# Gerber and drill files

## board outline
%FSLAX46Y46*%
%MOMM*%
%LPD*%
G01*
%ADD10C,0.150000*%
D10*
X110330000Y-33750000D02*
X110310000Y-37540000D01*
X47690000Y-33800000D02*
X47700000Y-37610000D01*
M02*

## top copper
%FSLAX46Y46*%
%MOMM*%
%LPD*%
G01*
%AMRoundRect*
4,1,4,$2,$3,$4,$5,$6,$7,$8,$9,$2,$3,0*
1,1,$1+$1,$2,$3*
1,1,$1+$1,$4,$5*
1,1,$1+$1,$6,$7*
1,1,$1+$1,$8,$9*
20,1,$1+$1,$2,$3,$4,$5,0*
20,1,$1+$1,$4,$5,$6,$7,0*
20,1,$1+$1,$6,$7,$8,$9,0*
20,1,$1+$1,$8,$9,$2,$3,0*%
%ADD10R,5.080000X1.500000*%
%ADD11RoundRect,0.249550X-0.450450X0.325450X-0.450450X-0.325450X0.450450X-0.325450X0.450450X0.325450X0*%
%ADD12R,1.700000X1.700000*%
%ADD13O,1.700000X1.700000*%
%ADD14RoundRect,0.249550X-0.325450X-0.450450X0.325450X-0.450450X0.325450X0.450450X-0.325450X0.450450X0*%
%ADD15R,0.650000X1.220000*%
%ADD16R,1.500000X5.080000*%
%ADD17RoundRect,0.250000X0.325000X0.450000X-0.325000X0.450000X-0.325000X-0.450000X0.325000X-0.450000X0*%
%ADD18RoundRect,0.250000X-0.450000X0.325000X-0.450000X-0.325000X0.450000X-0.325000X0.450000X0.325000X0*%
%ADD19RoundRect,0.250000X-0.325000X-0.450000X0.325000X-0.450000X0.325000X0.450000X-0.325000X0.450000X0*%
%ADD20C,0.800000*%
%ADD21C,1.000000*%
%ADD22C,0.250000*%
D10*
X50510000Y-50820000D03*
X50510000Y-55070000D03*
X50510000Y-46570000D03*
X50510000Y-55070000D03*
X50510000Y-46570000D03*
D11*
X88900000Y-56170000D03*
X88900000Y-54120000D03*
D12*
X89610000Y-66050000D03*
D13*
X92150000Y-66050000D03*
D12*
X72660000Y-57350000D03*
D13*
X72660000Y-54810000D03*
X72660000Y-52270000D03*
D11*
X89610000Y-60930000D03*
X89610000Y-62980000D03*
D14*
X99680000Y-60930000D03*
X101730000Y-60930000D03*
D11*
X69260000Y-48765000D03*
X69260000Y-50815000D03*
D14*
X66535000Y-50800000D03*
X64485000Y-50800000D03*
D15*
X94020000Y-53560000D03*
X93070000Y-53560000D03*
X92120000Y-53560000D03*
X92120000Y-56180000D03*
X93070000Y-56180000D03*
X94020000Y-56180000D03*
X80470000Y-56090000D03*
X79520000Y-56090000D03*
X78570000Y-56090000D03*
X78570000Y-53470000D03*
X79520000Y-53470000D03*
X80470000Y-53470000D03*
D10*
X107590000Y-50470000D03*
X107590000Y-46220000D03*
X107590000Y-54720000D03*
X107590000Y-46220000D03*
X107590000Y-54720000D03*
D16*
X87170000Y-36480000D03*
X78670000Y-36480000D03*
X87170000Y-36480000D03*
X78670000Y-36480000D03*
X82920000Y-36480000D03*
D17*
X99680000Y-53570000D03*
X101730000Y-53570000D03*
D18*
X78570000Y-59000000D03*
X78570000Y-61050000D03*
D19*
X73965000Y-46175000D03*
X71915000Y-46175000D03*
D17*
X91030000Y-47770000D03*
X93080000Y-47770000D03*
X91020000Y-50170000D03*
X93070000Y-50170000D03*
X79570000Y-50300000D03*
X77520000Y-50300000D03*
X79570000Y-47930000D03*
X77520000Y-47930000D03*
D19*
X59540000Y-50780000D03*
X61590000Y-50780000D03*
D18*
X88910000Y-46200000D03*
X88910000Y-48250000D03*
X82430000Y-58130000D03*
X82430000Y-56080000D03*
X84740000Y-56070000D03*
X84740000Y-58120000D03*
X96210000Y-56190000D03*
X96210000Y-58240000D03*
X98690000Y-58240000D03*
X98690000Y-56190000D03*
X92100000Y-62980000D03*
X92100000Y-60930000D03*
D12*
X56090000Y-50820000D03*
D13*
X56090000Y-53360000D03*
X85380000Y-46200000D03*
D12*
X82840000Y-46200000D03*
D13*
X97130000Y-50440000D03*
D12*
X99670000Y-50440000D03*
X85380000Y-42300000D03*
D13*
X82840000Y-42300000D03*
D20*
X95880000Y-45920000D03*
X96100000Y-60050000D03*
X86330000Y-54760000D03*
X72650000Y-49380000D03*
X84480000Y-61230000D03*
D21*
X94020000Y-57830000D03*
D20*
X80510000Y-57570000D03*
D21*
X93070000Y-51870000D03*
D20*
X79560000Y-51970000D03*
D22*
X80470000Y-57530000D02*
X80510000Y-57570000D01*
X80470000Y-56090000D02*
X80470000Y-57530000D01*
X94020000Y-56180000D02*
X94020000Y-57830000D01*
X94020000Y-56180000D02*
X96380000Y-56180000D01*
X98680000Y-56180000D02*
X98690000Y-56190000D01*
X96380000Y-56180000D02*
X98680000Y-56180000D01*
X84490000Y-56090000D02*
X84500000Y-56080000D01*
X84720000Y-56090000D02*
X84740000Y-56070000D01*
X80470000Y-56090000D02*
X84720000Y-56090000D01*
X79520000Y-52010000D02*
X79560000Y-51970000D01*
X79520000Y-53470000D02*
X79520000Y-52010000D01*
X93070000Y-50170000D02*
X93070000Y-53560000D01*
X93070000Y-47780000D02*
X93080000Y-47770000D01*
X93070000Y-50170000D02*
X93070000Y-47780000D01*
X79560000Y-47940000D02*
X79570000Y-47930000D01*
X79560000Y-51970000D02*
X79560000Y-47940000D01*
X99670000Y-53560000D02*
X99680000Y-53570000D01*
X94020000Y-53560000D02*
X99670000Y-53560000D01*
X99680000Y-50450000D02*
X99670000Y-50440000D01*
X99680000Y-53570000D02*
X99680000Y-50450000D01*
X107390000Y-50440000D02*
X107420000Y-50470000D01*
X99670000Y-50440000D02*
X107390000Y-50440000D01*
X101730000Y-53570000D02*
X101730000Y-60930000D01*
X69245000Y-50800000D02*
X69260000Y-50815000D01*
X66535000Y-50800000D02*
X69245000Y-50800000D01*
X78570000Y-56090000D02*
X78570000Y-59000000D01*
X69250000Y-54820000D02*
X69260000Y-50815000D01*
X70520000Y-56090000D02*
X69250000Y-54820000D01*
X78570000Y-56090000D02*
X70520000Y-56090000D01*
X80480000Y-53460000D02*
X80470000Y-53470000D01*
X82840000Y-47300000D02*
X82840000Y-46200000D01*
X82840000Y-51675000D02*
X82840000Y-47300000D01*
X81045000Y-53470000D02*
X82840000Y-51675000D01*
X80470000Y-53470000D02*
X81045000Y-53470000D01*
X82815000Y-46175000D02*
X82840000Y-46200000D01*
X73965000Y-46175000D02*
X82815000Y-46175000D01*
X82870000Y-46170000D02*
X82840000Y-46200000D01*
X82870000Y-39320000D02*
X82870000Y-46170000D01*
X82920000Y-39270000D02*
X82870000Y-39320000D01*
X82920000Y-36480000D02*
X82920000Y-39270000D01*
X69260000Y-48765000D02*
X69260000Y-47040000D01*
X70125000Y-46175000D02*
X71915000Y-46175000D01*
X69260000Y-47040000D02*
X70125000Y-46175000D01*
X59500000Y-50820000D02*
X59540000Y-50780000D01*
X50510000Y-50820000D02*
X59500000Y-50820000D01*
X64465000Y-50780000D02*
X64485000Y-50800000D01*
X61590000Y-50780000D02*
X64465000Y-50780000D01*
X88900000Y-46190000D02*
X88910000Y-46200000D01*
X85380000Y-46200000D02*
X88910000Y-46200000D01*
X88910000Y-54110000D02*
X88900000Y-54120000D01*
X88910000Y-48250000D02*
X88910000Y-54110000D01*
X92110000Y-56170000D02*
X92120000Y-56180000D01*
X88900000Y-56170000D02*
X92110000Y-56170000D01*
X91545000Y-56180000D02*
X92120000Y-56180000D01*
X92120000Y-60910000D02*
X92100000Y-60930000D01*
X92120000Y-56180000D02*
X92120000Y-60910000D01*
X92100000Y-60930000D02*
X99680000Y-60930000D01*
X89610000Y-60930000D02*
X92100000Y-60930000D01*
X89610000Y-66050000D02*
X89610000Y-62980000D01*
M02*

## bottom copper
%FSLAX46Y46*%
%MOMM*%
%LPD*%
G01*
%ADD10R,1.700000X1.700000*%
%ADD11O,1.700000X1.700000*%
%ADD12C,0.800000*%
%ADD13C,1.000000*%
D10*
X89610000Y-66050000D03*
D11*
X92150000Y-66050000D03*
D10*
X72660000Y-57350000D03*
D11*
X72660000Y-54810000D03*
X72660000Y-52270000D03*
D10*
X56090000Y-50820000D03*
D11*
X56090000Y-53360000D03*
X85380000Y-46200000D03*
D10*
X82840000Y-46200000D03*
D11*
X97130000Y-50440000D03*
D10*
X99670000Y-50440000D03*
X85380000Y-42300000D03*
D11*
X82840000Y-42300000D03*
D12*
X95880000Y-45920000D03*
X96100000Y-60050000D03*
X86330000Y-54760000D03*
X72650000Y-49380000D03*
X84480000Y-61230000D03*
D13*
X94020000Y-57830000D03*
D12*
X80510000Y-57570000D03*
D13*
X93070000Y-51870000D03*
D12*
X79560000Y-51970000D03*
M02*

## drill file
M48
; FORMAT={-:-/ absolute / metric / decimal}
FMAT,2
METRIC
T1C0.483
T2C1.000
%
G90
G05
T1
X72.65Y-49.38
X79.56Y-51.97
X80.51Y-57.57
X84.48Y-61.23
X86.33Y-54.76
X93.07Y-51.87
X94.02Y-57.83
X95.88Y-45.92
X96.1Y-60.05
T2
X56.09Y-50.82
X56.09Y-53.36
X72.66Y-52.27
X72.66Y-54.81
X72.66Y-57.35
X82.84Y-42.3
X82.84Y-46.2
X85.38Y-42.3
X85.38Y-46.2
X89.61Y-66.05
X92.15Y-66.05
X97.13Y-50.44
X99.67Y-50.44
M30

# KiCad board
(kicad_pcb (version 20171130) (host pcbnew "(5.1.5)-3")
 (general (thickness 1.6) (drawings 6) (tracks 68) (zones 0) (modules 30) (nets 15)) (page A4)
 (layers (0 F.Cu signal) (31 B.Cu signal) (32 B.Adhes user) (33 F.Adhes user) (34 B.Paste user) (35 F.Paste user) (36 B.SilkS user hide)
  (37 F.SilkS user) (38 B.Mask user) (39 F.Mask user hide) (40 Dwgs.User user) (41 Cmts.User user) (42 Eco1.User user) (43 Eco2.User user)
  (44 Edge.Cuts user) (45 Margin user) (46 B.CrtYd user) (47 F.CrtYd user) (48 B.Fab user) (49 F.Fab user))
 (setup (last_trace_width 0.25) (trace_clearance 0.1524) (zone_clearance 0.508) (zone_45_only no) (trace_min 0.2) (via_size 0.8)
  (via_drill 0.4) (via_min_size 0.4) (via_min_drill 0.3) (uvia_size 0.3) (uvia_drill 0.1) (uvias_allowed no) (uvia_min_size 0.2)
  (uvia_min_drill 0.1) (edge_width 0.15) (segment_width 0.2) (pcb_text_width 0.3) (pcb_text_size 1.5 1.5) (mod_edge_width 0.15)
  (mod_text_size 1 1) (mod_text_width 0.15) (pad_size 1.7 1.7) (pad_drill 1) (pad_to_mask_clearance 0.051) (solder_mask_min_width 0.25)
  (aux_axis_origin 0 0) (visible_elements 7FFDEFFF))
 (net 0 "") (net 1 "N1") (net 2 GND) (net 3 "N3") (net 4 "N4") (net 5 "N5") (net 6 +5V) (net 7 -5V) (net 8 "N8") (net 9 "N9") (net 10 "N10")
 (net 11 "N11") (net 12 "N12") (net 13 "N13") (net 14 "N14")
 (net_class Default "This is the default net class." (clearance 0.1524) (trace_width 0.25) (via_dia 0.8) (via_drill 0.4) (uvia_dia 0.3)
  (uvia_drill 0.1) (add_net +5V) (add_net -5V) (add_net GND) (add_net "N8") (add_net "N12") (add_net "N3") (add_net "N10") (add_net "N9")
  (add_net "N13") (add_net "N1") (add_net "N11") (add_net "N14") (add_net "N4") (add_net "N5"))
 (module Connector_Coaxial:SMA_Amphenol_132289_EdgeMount (layer F.Cu) (at 50.51 50.82 180)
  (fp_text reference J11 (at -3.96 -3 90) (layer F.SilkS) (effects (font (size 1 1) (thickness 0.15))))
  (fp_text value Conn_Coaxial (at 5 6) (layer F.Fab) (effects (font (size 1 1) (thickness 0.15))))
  (pad 1 smd rect (at 0 0 270) (size 1.5 5.08) (layers F.Cu F.Paste F.Mask) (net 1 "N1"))
  (pad 2 smd rect (at 0 -4.25 270) (size 1.5 5.08) (layers F.Cu F.Paste F.Mask) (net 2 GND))
  (pad 2 smd rect (at 0 4.25 270) (size 1.5 5.08) (layers F.Cu F.Paste F.Mask) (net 2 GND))
  (pad 2 smd rect (at 0 -4.25 270) (size 1.5 5.08) (layers F.Cu B.Paste B.Mask) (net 2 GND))
  (pad 2 smd rect (at 0 4.25 270) (size 1.5 5.08) (layers F.Cu B.Paste B.Mask) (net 2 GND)))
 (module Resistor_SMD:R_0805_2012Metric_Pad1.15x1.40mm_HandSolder (layer F.Cu) (at 88.9 55.145 270)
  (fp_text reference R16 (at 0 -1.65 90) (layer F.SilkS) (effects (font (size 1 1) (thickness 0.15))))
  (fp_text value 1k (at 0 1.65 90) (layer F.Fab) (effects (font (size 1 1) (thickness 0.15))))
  (pad 2 smd roundrect (at 1.025 0 270) (size 1.15 1.4) (layers F.Cu F.Paste F.Mask) (roundrect_rratio 0.217) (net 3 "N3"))
  (pad 1 smd roundrect (at -1.025 0 270) (size 1.15 1.4) (layers F.Cu F.Paste F.Mask) (roundrect_rratio 0.217) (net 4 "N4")))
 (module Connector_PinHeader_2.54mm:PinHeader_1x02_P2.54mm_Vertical (layer F.Cu) (at 89.61 66.05 90)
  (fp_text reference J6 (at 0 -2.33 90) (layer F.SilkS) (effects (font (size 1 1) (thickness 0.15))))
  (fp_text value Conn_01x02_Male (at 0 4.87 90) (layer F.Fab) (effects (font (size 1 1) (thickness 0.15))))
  (pad 1 thru_hole rect (at 0 0 90) (size 1.7 1.7) (drill 1) (layers *.Cu *.Mask) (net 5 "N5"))
  (pad 2 thru_hole oval (at 0 2.54 90) (size 1.7 1.7) (drill 1) (layers *.Cu *.Mask) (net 2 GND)))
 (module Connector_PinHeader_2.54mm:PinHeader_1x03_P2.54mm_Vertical (layer F.Cu) (at 72.66 57.35 180)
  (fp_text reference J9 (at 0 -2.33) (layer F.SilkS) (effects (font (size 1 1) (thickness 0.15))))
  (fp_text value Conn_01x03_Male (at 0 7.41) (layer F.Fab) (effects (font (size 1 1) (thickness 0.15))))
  (pad 1 thru_hole rect (at 0 0 180) (size 1.7 1.7) (drill 1) (layers *.Mask B.Cu) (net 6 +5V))
  (pad 2 thru_hole oval (at 0 2.54 180) (size 1.7 1.7) (drill 1) (layers *.Cu *.Mask) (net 2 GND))
  (pad 3 thru_hole oval (at 0 5.08 180) (size 1.7 1.7) (drill 1) (layers *.Mask B.Cu) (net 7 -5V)))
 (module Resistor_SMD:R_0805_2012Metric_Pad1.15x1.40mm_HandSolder (layer F.Cu) (at 89.61 61.955 270)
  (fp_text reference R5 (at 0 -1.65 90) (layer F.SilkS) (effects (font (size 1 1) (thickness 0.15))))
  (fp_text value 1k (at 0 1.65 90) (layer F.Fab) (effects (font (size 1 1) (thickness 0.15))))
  (pad 1 smd roundrect (at -1.025 0 270) (size 1.15 1.4) (layers F.Cu F.Paste F.Mask) (roundrect_rratio 0.217) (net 3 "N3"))
  (pad 2 smd roundrect (at 1.025 0 270) (size 1.15 1.4) (layers F.Cu F.Paste F.Mask) (roundrect_rratio 0.217) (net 5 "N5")))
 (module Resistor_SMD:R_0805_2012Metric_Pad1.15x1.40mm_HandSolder (layer F.Cu) (at 100.705 60.93)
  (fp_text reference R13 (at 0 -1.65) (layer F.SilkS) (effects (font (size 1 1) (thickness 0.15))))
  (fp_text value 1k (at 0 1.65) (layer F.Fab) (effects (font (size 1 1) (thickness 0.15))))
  (pad 1 smd roundrect (at -1.025 0) (size 1.15 1.4) (layers F.Cu F.Paste F.Mask) (roundrect_rratio 0.217) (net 3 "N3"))
  (pad 2 smd roundrect (at 1.025 0) (size 1.15 1.4) (layers F.Cu F.Paste F.Mask) (roundrect_rratio 0.217) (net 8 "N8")))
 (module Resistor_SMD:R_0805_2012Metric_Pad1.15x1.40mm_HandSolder (layer F.Cu) (at 69.26 49.79 270)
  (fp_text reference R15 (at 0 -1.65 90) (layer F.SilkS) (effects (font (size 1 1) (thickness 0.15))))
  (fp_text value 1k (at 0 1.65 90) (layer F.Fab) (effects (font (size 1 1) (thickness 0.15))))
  (pad 1 smd roundrect (at -1.025 0 270) (size 1.15 1.4) (layers F.Cu F.Paste F.Mask) (roundrect_rratio 0.217) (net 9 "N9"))
  (pad 2 smd roundrect (at 1.025 0 270) (size 1.15 1.4) (layers F.Cu F.Paste F.Mask) (roundrect_rratio 0.217) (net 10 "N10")))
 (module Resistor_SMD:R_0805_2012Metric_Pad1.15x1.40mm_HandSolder (layer F.Cu) (at 65.51 50.8)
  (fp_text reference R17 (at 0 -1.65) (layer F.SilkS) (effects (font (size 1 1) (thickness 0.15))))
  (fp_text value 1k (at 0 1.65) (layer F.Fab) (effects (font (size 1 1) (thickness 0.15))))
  (pad 2 smd roundrect (at 1.025 0) (size 1.15 1.4) (layers F.Cu F.Paste F.Mask) (roundrect_rratio 0.217) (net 10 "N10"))
  (pad 1 smd roundrect (at -1.025 0) (size 1.15 1.4) (layers F.Cu F.Paste F.Mask) (roundrect_rratio 0.217) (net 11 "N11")))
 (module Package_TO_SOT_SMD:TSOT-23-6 (layer F.Cu) (at 93.07 54.87 270)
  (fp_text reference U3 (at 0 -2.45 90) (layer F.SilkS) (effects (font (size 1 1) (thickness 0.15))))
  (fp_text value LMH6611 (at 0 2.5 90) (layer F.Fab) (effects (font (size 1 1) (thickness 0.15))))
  (pad 1 smd rect (at -1.31 -0.95 270) (size 1.22 0.65) (layers F.Cu F.Paste F.Mask) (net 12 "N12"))
  (pad 2 smd rect (at -1.31 0 270) (size 1.22 0.65) (layers F.Cu F.Paste F.Mask) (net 7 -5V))
  (pad 3 smd rect (at -1.31 0.95 270) (size 1.22 0.65) (layers F.Cu F.Paste F.Mask) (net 2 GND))
  (pad 4 smd rect (at 1.31 0.95 270) (size 1.22 0.65) (layers F.Cu F.Paste F.Mask) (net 3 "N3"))
  (pad 5 smd rect (at 1.31 0 270) (size 1.22 0.65) (layers F.Cu F.Paste F.Mask))
  (pad 6 smd rect (at 1.31 -0.95 270) (size 1.22 0.65) (layers F.Cu F.Paste F.Mask) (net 6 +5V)))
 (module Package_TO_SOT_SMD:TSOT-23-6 (layer F.Cu) (at 79.52 54.78 270)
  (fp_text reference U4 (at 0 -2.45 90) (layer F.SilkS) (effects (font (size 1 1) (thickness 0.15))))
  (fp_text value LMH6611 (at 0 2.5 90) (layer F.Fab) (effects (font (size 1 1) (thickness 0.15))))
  (pad 6 smd rect (at 1.31 -0.95 270) (size 1.22 0.65) (layers F.Cu F.Paste F.Mask) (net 6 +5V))
  (pad 5 smd rect (at 1.31 0 270) (size 1.22 0.65) (layers F.Cu F.Paste F.Mask))
  (pad 4 smd rect (at 1.31 0.95 270) (size 1.22 0.65) (layers F.Cu F.Paste F.Mask) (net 10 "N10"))
  (pad 3 smd rect (at -1.31 0.95 270) (size 1.22 0.65) (layers F.Cu F.Paste F.Mask) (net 2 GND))
  (pad 2 smd rect (at -1.31 0 270) (size 1.22 0.65) (layers F.Cu F.Paste F.Mask) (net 7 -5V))
  (pad 1 smd rect (at -1.31 -0.95 270) (size 1.22 0.65) (layers F.Cu F.Paste F.Mask) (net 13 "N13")))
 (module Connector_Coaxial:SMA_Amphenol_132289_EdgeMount (layer F.Cu) (at 107.59 50.47)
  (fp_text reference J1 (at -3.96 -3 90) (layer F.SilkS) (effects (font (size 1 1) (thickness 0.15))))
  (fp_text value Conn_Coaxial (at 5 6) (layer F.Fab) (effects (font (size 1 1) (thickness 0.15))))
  (pad 1 smd rect (at 0 0 90) (size 1.5 5.08) (layers F.Cu F.Paste F.Mask) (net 12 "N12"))
  (pad 2 smd rect (at 0 -4.25 90) (size 1.5 5.08) (layers F.Cu F.Paste F.Mask) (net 2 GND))
  (pad 2 smd rect (at 0 4.25 90) (size 1.5 5.08) (layers F.Cu F.Paste F.Mask) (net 2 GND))
  (pad 2 smd rect (at 0 -4.25 90) (size 1.5 5.08) (layers F.Cu B.Paste B.Mask) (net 2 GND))
  (pad 2 smd rect (at 0 4.25 90) (size 1.5 5.08) (layers F.Cu B.Paste B.Mask) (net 2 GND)))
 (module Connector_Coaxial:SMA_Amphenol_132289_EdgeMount (layer F.Cu) (at 82.92 36.48 90)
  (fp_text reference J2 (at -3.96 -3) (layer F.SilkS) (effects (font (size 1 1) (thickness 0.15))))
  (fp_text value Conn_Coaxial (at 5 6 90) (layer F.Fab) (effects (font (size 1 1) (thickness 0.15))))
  (pad 2 smd rect (at 0 4.25 180) (size 1.5 5.08) (layers F.Cu B.Paste B.Mask) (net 2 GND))
  (pad 2 smd rect (at 0 -4.25 180) (size 1.5 5.08) (layers F.Cu B.Paste B.Mask) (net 2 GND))
  (pad 2 smd rect (at 0 4.25 180) (size 1.5 5.08) (layers F.Cu F.Paste F.Mask) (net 2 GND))
  (pad 2 smd rect (at 0 -4.25 180) (size 1.5 5.08) (layers F.Cu F.Paste F.Mask) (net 2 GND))
  (pad 1 smd rect (at 0 0 180) (size 1.5 5.08) (layers F.Cu F.Paste F.Mask) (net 13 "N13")))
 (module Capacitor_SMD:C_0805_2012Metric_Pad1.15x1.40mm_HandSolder (layer F.Cu) (at 100.705 53.57 180)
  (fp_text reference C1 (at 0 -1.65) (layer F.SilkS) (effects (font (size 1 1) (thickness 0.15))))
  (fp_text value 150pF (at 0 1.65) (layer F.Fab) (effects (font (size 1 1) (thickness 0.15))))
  (pad 2 smd roundrect (at 1.025 0 180) (size 1.15 1.4) (layers F.Cu F.Paste F.Mask) (roundrect_rratio 0.217391) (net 12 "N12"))
  (pad 1 smd roundrect (at -1.025 0 180) (size 1.15 1.4) (layers F.Cu F.Paste F.Mask) (roundrect_rratio 0.217391) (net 8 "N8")))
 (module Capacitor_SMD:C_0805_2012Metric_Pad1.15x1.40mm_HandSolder (layer F.Cu) (at 78.57 60.025 270)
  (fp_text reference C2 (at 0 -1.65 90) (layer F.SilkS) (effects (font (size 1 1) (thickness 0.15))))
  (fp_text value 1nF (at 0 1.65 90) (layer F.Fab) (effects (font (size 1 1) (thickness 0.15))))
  (pad 1 smd roundrect (at -1.025 0 270) (size 1.15 1.4) (layers F.Cu F.Paste F.Mask) (roundrect_rratio 0.217391) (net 10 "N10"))
  (pad 2 smd roundrect (at 1.025 0 270) (size 1.15 1.4) (layers F.Cu F.Paste F.Mask) (roundrect_rratio 0.217391) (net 2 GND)))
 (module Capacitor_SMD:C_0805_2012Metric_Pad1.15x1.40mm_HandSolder (layer F.Cu) (at 72.94 46.175)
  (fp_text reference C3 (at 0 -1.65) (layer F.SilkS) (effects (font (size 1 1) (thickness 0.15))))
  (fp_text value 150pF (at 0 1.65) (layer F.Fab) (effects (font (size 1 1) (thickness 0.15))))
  (pad 2 smd roundrect (at 1.025 0) (size 1.15 1.4) (layers F.Cu F.Paste F.Mask) (roundrect_rratio 0.217391) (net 13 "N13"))
  (pad 1 smd roundrect (at -1.025 0) (size 1.15 1.4) (layers F.Cu F.Paste F.Mask) (roundrect_rratio 0.217391) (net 9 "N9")))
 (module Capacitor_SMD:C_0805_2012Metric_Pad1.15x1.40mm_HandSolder (layer F.Cu) (at 92.055 47.77 180)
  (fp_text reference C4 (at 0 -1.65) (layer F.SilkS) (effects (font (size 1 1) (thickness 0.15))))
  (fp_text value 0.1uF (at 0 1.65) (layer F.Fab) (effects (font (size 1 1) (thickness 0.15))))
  (pad 2 smd roundrect (at 1.025 0 180) (size 1.15 1.4) (layers F.Cu F.Paste F.Mask) (roundrect_rratio 0.217391) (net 2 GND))
  (pad 1 smd roundrect (at -1.025 0 180) (size 1.15 1.4) (layers F.Cu F.Paste F.Mask) (roundrect_rratio 0.217391) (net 7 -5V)))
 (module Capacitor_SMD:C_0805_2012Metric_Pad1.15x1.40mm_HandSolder (layer F.Cu) (at 92.045 50.17 180)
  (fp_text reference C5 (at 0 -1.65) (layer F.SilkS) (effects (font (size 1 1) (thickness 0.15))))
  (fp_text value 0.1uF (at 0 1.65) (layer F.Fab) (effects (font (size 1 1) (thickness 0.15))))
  (pad 2 smd roundrect (at 1.025 0 180) (size 1.15 1.4) (layers F.Cu F.Paste F.Mask) (roundrect_rratio 0.217391) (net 2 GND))
  (pad 1 smd roundrect (at -1.025 0 180) (size 1.15 1.4) (layers F.Cu F.Paste F.Mask) (roundrect_rratio 0.217391) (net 7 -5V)))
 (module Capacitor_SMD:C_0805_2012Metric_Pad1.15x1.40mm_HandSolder (layer F.Cu) (at 78.545 50.3 180)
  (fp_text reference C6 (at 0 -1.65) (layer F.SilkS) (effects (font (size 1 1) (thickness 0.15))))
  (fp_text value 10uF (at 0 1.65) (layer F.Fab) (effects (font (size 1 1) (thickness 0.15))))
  (pad 1 smd roundrect (at -1.025 0 180) (size 1.15 1.4) (layers F.Cu F.Paste F.Mask) (roundrect_rratio 0.217391) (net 7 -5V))
  (pad 2 smd roundrect (at 1.025 0 180) (size 1.15 1.4) (layers F.Cu F.Paste F.Mask) (roundrect_rratio 0.217391) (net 2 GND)))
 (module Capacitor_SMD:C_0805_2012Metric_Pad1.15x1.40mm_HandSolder (layer F.Cu) (at 78.545 47.93 180)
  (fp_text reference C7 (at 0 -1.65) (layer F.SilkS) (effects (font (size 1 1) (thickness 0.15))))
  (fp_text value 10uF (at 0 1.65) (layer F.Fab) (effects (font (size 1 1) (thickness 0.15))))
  (pad 1 smd roundrect (at -1.025 0 180) (size 1.15 1.4) (layers F.Cu F.Paste F.Mask) (roundrect_rratio 0.217391) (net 7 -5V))
  (pad 2 smd roundrect (at 1.025 0 180) (size 1.15 1.4) (layers F.Cu F.Paste F.Mask) (roundrect_rratio 0.217391) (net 2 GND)))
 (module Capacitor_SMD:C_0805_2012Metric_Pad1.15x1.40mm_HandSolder (layer F.Cu) (at 60.565 50.78)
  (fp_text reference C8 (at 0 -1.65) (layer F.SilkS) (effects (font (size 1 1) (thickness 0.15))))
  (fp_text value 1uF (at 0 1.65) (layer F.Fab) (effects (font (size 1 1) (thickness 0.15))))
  (pad 1 smd roundrect (at -1.025 0) (size 1.15 1.4) (layers F.Cu F.Paste F.Mask) (roundrect_rratio 0.217391) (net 1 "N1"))
  (pad 2 smd roundrect (at 1.025 0) (size 1.15 1.4) (layers F.Cu F.Paste F.Mask) (roundrect_rratio 0.217391) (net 11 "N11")))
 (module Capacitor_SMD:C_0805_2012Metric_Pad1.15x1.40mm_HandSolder (layer F.Cu) (at 88.91 47.225 270)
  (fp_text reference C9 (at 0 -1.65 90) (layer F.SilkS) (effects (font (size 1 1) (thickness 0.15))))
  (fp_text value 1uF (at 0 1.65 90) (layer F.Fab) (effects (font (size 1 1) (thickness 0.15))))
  (pad 1 smd roundrect (at -1.025 0 270) (size 1.15 1.4) (layers F.Cu F.Paste F.Mask) (roundrect_rratio 0.217391) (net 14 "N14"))
  (pad 2 smd roundrect (at 1.025 0 270) (size 1.15 1.4) (layers F.Cu F.Paste F.Mask) (roundrect_rratio 0.217391) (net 4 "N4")))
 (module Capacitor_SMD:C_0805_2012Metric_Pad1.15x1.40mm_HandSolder (layer F.Cu) (at 82.43 57.105 270)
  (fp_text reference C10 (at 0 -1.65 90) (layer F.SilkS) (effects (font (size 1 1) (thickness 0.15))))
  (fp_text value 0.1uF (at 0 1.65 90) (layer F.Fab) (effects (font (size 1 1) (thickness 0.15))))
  (pad 2 smd roundrect (at 1.025 0 270) (size 1.15 1.4) (layers F.Cu F.Paste F.Mask) (roundrect_rratio 0.217391) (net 2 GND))
  (pad 1 smd roundrect (at -1.025 0 270) (size 1.15 1.4) (layers F.Cu F.Paste F.Mask) (roundrect_rratio 0.217391) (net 6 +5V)))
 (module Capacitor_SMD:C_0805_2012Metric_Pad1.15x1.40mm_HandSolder (layer F.Cu) (at 84.74 57.095 270)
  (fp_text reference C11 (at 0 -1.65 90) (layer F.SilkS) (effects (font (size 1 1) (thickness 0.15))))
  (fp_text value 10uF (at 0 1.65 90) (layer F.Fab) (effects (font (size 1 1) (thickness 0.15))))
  (pad 1 smd roundrect (at -1.025 0 270) (size 1.15 1.4) (layers F.Cu F.Paste F.Mask) (roundrect_rratio 0.217391) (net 6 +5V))
  (pad 2 smd roundrect (at 1.025 0 270) (size 1.15 1.4) (layers F.Cu F.Paste F.Mask) (roundrect_rratio 0.217391) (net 2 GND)))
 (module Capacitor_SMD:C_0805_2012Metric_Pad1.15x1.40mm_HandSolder (layer F.Cu) (at 96.21 57.215 270)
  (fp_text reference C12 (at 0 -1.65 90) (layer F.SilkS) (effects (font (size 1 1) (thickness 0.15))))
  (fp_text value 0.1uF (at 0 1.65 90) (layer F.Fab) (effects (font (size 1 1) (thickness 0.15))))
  (pad 1 smd roundrect (at -1.025 0 270) (size 1.15 1.4) (layers F.Cu F.Paste F.Mask) (roundrect_rratio 0.217391) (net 6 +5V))
  (pad 2 smd roundrect (at 1.025 0 270) (size 1.15 1.4) (layers F.Cu F.Paste F.Mask) (roundrect_rratio 0.217391) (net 2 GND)))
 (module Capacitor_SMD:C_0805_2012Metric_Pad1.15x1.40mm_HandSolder (layer F.Cu) (at 98.69 57.215 270)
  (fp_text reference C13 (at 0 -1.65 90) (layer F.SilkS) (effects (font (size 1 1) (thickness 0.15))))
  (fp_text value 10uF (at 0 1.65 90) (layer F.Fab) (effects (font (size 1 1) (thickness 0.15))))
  (pad 2 smd roundrect (at 1.025 0 270) (size 1.15 1.4) (layers F.Cu F.Paste F.Mask) (roundrect_rratio 0.217391) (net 2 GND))
  (pad 1 smd roundrect (at -1.025 0 270) (size 1.15 1.4) (layers F.Cu F.Paste F.Mask) (roundrect_rratio 0.217391) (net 6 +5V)))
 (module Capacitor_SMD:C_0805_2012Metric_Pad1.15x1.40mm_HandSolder (layer F.Cu) (at 92.1 61.955 270)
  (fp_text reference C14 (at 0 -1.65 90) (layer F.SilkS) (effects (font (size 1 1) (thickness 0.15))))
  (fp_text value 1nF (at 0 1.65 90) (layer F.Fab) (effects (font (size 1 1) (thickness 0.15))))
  (pad 2 smd roundrect (at 1.025 0 270) (size 1.15 1.4) (layers F.Cu F.Paste F.Mask) (roundrect_rratio 0.217391) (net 2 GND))
  (pad 1 smd roundrect (at -1.025 0 270) (size 1.15 1.4) (layers F.Cu F.Paste F.Mask) (roundrect_rratio 0.217391) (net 3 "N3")))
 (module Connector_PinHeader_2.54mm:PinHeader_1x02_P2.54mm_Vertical (layer F.Cu) (at 56.09 50.82)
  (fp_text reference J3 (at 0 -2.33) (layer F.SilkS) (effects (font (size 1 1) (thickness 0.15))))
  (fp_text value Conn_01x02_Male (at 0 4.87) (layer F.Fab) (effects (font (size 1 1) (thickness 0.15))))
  (pad 1 thru_hole rect (at 0 0) (size 1.7 1.7) (drill 1) (layers *.Cu *.Mask) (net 1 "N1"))
  (pad 2 thru_hole oval (at 0 2.54) (size 1.7 1.7) (drill 1) (layers *.Cu *.Mask) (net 2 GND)))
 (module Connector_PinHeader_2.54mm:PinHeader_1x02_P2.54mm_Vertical (layer F.Cu) (at 82.84 46.2 90)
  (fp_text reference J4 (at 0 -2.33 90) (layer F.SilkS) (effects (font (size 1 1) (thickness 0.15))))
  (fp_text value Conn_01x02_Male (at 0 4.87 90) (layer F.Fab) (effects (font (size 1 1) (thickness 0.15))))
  (pad 2 thru_hole oval (at 0 2.54 90) (size 1.7 1.7) (drill 1) (layers *.Cu *.Mask) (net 14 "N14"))
  (pad 1 thru_hole rect (at 0 0 90) (size 1.7 1.7) (drill 1) (layers *.Cu *.Mask) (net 13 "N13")))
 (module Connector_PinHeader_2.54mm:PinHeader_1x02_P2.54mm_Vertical (layer F.Cu) (at 99.67 50.44 270)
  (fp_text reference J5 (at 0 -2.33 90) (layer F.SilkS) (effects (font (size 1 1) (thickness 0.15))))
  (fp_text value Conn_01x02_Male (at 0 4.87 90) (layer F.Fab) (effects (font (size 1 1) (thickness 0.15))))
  (pad 2 thru_hole oval (at 0 2.54 270) (size 1.7 1.7) (drill 1) (layers *.Cu *.Mask) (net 2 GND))
  (pad 1 thru_hole rect (at 0 0 270) (size 1.7 1.7) (drill 1) (layers *.Cu *.Mask) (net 12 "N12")))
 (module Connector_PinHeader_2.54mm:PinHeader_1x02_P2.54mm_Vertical (layer F.Cu) (at 85.38 42.3 270)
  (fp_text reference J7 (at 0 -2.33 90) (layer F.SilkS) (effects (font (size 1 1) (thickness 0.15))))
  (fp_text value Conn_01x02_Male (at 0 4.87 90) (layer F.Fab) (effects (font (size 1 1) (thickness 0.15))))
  (pad 1 thru_hole rect (at 0 0 270) (size 1.7 1.7) (drill 1) (layers *.Cu *.Mask) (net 2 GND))
  (pad 2 thru_hole oval (at 0 2.54 270) (size 1.7 1.7) (drill 1) (layers *.Cu *.Mask) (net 13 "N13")))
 (gr_line (start 110.33 33.75) (end 110.31 37.54) (layer Edge.Cuts) (width 0.15))
 (gr_line (start 47.69 33.8) (end 47.7 37.61) (layer Edge.Cuts) (width 0.15))
 (via (at 95.88 45.92) (size 0.8) (drill 0.4826) (layers F.Cu B.Cu) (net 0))
 (via (at 96.1 60.05) (size 0.8) (drill 0.4826) (layers F.Cu B.Cu) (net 2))
 (via (at 86.33 54.76) (size 0.8) (drill 0.4826) (layers F.Cu B.Cu) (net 2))
 (via (at 72.65 49.38) (size 0.8) (drill 0.4826) (layers F.Cu B.Cu) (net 2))
 (via (at 84.48 61.23) (size 0.8) (drill 0.4826) (layers F.Cu B.Cu) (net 2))
 (via (at 94.02 57.83) (size 1) (drill 0.4826) (layers F.Cu B.Cu) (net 6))
 (via (at 80.51 57.57) (size 0.8) (drill 0.4826) (layers F.Cu B.Cu) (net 6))
 (segment (start 80.47 57.53) (end 80.51 57.57) (width 0.25) (layer F.Cu) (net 6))
 (segment (start 80.47 56.09) (end 80.47 57.53) (width 0.25) (layer F.Cu) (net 6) (status 10))
 (segment (start 94.02 56.18) (end 94.02 57.83) (width 0.25) (layer F.Cu) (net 6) (status 10))
 (segment (start 94.02 56.18) (end 96.38 56.18) (width 0.25) (layer F.Cu) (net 6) (status 30))
 (segment (start 98.68 56.18) (end 98.69 56.19) (width 0.25) (layer F.Cu) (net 6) (status 30))
 (segment (start 96.38 56.18) (end 98.68 56.18) (width 0.25) (layer F.Cu) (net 6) (status 30))
 (segment (start 84.49 56.09) (end 84.5 56.08) (width 0.25) (layer F.Cu) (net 6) (status 30))
 (segment (start 84.72 56.09) (end 84.74 56.07) (width 0.25) (layer F.Cu) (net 6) (status 30))
 (segment (start 80.47 56.09) (end 84.72 56.09) (width 0.25) (layer F.Cu) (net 6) (status 30))
 (via (at 93.07 51.87) (size 1) (drill 0.4826) (layers F.Cu B.Cu) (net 7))
 (via (at 79.56 51.97) (size 0.8) (drill 0.4826) (layers F.Cu B.Cu) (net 7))
 (segment (start 79.52 52.01) (end 79.56 51.97) (width 0.25) (layer F.Cu) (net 7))
 (segment (start 79.52 53.47) (end 79.52 52.01) (width 0.25) (layer F.Cu) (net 7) (status 10))
 (segment (start 93.07 50.17) (end 93.07 53.56) (width 0.25) (layer F.Cu) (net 7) (status 30))
 (segment (start 93.07 47.78) (end 93.08 47.77) (width 0.25) (layer F.Cu) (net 7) (status 30))
 (segment (start 93.07 50.17) (end 93.07 47.78) (width 0.25) (layer F.Cu) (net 7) (status 30))
 (segment (start 79.56 47.94) (end 79.57 47.93) (width 0.25) (layer F.Cu) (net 7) (status 30))
 (segment (start 79.56 51.97) (end 79.56 47.94) (width 0.25) (layer F.Cu) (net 7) (status 20))
 (segment (start 99.67 53.56) (end 99.68 53.57) (width 0.25) (layer F.Cu) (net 12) (status 30))
 (segment (start 94.02 53.56) (end 99.67 53.56) (width 0.25) (layer F.Cu) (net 12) (status 30))
 (segment (start 99.68 50.45) (end 99.67 50.44) (width 0.25) (layer F.Cu) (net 12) (status 30))
 (segment (start 99.68 53.57) (end 99.68 50.45) (width 0.25) (layer F.Cu) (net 12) (status 30))
 (segment (start 107.39 50.44) (end 107.42 50.47) (width 0.25) (layer F.Cu) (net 12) (status 30))
 (segment (start 99.67 50.44) (end 107.39 50.44) (width 0.25) (layer F.Cu) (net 12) (status 30))
 (segment (start 101.73 53.57) (end 101.73 60.93) (width 0.25) (layer F.Cu) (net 8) (status 30))
 (segment (start 69.245 50.8) (end 69.26 50.815) (width 0.25) (layer F.Cu) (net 10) (status 30))
 (segment (start 66.535 50.8) (end 69.245 50.8) (width 0.25) (layer F.Cu) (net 10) (status 30))
 (segment (start 78.57 56.09) (end 78.57 59) (width 0.25) (layer F.Cu) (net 10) (status 30))
 (segment (start 69.25 54.82) (end 69.26 50.815) (width 0.25) (layer F.Cu) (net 10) (status 20))
 (segment (start 70.52 56.09) (end 69.25 54.82) (width 0.25) (layer F.Cu) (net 10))
 (segment (start 78.57 56.09) (end 70.52 56.09) (width 0.25) (layer F.Cu) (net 10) (status 10))
 (segment (start 80.48 53.46) (end 80.47 53.47) (width 0.25) (layer F.Cu) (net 13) (status 30))
 (segment (start 82.84 47.3) (end 82.84 46.2) (width 0.25) (layer F.Cu) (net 13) (status 20))
 (segment (start 82.84 51.675) (end 82.84 47.3) (width 0.25) (layer F.Cu) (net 13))
 (segment (start 81.045 53.47) (end 82.84 51.675) (width 0.25) (layer F.Cu) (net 13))
 (segment (start 80.47 53.47) (end 81.045 53.47) (width 0.25) (layer F.Cu) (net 13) (status 10))
 (segment (start 82.815 46.175) (end 82.84 46.2) (width 0.25) (layer F.Cu) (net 13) (status 30))
 (segment (start 73.965 46.175) (end 82.815 46.175) (width 0.25) (layer F.Cu) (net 13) (status 30))
 (segment (start 82.87 46.17) (end 82.84 46.2) (width 0.25) (layer F.Cu) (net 13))
 (segment (start 82.87 39.32) (end 82.87 46.17) (width 0.25) (layer F.Cu) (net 13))
 (segment (start 82.92 39.27) (end 82.87 39.32) (width 0.25) (layer F.Cu) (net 13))
 (segment (start 82.92 36.48) (end 82.92 39.27) (width 0.25) (layer F.Cu) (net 13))
 (segment (start 69.26 48.765) (end 69.26 47.04) (width 0.25) (layer F.Cu) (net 9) (status 10))
 (segment (start 70.125 46.175) (end 71.915 46.175) (width 0.25) (layer F.Cu) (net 9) (status 20))
 (segment (start 69.26 47.04) (end 70.125 46.175) (width 0.25) (layer F.Cu) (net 9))
 (segment (start 59.5 50.82) (end 59.54 50.78) (width 0.25) (layer F.Cu) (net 1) (status 30))
 (segment (start 50.51 50.82) (end 59.5 50.82) (width 0.25) (layer F.Cu) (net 1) (status 30))
 (segment (start 64.465 50.78) (end 64.485 50.8) (width 0.25) (layer F.Cu) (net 11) (status 30))
 (segment (start 61.59 50.78) (end 64.465 50.78) (width 0.25) (layer F.Cu) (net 11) (status 30))
 (segment (start 88.9 46.19) (end 88.91 46.2) (width 0.25) (layer F.Cu) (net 14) (status 30))
 (segment (start 85.38 46.2) (end 88.91 46.2) (width 0.25) (layer F.Cu) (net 14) (status 30))
 (segment (start 88.91 54.11) (end 88.9 54.12) (width 0.25) (layer F.Cu) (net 4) (status 30))
 (segment (start 88.91 48.25) (end 88.91 54.11) (width 0.25) (layer F.Cu) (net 4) (status 30))
 (segment (start 92.11 56.17) (end 92.12 56.18) (width 0.25) (layer F.Cu) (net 3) (status 30))
 (segment (start 88.9 56.17) (end 92.11 56.17) (width 0.25) (layer F.Cu) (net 3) (status 30))
 (segment (start 91.545 56.18) (end 92.12 56.18) (width 0.25) (layer F.Cu) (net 3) (status 20))
 (segment (start 92.12 60.91) (end 92.1 60.93) (width 0.25) (layer F.Cu) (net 3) (status 30))
 (segment (start 92.12 56.18) (end 92.12 60.91) (width 0.25) (layer F.Cu) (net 3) (status 30))
 (segment (start 92.1 60.93) (end 99.68 60.93) (width 0.25) (layer F.Cu) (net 3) (status 30))
 (segment (start 89.61 60.93) (end 92.1 60.93) (width 0.25) (layer F.Cu) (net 3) (status 30))
 (segment (start 89.61 66.05) (end 89.61 62.98) (width 0.25) (layer F.Cu) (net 5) (status 30))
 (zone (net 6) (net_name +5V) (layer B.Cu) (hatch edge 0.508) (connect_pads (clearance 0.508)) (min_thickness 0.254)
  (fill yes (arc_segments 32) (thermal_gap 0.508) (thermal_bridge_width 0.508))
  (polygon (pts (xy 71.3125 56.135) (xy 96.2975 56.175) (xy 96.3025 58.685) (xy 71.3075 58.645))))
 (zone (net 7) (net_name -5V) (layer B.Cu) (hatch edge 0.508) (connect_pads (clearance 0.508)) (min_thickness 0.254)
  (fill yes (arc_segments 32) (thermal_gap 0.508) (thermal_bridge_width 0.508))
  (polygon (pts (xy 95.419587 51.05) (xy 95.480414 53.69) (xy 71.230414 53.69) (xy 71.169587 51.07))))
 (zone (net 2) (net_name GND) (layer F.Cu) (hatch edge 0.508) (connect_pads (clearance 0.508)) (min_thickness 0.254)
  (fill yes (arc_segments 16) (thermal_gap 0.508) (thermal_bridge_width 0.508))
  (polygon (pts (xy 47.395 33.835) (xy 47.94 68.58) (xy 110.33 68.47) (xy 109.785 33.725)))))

